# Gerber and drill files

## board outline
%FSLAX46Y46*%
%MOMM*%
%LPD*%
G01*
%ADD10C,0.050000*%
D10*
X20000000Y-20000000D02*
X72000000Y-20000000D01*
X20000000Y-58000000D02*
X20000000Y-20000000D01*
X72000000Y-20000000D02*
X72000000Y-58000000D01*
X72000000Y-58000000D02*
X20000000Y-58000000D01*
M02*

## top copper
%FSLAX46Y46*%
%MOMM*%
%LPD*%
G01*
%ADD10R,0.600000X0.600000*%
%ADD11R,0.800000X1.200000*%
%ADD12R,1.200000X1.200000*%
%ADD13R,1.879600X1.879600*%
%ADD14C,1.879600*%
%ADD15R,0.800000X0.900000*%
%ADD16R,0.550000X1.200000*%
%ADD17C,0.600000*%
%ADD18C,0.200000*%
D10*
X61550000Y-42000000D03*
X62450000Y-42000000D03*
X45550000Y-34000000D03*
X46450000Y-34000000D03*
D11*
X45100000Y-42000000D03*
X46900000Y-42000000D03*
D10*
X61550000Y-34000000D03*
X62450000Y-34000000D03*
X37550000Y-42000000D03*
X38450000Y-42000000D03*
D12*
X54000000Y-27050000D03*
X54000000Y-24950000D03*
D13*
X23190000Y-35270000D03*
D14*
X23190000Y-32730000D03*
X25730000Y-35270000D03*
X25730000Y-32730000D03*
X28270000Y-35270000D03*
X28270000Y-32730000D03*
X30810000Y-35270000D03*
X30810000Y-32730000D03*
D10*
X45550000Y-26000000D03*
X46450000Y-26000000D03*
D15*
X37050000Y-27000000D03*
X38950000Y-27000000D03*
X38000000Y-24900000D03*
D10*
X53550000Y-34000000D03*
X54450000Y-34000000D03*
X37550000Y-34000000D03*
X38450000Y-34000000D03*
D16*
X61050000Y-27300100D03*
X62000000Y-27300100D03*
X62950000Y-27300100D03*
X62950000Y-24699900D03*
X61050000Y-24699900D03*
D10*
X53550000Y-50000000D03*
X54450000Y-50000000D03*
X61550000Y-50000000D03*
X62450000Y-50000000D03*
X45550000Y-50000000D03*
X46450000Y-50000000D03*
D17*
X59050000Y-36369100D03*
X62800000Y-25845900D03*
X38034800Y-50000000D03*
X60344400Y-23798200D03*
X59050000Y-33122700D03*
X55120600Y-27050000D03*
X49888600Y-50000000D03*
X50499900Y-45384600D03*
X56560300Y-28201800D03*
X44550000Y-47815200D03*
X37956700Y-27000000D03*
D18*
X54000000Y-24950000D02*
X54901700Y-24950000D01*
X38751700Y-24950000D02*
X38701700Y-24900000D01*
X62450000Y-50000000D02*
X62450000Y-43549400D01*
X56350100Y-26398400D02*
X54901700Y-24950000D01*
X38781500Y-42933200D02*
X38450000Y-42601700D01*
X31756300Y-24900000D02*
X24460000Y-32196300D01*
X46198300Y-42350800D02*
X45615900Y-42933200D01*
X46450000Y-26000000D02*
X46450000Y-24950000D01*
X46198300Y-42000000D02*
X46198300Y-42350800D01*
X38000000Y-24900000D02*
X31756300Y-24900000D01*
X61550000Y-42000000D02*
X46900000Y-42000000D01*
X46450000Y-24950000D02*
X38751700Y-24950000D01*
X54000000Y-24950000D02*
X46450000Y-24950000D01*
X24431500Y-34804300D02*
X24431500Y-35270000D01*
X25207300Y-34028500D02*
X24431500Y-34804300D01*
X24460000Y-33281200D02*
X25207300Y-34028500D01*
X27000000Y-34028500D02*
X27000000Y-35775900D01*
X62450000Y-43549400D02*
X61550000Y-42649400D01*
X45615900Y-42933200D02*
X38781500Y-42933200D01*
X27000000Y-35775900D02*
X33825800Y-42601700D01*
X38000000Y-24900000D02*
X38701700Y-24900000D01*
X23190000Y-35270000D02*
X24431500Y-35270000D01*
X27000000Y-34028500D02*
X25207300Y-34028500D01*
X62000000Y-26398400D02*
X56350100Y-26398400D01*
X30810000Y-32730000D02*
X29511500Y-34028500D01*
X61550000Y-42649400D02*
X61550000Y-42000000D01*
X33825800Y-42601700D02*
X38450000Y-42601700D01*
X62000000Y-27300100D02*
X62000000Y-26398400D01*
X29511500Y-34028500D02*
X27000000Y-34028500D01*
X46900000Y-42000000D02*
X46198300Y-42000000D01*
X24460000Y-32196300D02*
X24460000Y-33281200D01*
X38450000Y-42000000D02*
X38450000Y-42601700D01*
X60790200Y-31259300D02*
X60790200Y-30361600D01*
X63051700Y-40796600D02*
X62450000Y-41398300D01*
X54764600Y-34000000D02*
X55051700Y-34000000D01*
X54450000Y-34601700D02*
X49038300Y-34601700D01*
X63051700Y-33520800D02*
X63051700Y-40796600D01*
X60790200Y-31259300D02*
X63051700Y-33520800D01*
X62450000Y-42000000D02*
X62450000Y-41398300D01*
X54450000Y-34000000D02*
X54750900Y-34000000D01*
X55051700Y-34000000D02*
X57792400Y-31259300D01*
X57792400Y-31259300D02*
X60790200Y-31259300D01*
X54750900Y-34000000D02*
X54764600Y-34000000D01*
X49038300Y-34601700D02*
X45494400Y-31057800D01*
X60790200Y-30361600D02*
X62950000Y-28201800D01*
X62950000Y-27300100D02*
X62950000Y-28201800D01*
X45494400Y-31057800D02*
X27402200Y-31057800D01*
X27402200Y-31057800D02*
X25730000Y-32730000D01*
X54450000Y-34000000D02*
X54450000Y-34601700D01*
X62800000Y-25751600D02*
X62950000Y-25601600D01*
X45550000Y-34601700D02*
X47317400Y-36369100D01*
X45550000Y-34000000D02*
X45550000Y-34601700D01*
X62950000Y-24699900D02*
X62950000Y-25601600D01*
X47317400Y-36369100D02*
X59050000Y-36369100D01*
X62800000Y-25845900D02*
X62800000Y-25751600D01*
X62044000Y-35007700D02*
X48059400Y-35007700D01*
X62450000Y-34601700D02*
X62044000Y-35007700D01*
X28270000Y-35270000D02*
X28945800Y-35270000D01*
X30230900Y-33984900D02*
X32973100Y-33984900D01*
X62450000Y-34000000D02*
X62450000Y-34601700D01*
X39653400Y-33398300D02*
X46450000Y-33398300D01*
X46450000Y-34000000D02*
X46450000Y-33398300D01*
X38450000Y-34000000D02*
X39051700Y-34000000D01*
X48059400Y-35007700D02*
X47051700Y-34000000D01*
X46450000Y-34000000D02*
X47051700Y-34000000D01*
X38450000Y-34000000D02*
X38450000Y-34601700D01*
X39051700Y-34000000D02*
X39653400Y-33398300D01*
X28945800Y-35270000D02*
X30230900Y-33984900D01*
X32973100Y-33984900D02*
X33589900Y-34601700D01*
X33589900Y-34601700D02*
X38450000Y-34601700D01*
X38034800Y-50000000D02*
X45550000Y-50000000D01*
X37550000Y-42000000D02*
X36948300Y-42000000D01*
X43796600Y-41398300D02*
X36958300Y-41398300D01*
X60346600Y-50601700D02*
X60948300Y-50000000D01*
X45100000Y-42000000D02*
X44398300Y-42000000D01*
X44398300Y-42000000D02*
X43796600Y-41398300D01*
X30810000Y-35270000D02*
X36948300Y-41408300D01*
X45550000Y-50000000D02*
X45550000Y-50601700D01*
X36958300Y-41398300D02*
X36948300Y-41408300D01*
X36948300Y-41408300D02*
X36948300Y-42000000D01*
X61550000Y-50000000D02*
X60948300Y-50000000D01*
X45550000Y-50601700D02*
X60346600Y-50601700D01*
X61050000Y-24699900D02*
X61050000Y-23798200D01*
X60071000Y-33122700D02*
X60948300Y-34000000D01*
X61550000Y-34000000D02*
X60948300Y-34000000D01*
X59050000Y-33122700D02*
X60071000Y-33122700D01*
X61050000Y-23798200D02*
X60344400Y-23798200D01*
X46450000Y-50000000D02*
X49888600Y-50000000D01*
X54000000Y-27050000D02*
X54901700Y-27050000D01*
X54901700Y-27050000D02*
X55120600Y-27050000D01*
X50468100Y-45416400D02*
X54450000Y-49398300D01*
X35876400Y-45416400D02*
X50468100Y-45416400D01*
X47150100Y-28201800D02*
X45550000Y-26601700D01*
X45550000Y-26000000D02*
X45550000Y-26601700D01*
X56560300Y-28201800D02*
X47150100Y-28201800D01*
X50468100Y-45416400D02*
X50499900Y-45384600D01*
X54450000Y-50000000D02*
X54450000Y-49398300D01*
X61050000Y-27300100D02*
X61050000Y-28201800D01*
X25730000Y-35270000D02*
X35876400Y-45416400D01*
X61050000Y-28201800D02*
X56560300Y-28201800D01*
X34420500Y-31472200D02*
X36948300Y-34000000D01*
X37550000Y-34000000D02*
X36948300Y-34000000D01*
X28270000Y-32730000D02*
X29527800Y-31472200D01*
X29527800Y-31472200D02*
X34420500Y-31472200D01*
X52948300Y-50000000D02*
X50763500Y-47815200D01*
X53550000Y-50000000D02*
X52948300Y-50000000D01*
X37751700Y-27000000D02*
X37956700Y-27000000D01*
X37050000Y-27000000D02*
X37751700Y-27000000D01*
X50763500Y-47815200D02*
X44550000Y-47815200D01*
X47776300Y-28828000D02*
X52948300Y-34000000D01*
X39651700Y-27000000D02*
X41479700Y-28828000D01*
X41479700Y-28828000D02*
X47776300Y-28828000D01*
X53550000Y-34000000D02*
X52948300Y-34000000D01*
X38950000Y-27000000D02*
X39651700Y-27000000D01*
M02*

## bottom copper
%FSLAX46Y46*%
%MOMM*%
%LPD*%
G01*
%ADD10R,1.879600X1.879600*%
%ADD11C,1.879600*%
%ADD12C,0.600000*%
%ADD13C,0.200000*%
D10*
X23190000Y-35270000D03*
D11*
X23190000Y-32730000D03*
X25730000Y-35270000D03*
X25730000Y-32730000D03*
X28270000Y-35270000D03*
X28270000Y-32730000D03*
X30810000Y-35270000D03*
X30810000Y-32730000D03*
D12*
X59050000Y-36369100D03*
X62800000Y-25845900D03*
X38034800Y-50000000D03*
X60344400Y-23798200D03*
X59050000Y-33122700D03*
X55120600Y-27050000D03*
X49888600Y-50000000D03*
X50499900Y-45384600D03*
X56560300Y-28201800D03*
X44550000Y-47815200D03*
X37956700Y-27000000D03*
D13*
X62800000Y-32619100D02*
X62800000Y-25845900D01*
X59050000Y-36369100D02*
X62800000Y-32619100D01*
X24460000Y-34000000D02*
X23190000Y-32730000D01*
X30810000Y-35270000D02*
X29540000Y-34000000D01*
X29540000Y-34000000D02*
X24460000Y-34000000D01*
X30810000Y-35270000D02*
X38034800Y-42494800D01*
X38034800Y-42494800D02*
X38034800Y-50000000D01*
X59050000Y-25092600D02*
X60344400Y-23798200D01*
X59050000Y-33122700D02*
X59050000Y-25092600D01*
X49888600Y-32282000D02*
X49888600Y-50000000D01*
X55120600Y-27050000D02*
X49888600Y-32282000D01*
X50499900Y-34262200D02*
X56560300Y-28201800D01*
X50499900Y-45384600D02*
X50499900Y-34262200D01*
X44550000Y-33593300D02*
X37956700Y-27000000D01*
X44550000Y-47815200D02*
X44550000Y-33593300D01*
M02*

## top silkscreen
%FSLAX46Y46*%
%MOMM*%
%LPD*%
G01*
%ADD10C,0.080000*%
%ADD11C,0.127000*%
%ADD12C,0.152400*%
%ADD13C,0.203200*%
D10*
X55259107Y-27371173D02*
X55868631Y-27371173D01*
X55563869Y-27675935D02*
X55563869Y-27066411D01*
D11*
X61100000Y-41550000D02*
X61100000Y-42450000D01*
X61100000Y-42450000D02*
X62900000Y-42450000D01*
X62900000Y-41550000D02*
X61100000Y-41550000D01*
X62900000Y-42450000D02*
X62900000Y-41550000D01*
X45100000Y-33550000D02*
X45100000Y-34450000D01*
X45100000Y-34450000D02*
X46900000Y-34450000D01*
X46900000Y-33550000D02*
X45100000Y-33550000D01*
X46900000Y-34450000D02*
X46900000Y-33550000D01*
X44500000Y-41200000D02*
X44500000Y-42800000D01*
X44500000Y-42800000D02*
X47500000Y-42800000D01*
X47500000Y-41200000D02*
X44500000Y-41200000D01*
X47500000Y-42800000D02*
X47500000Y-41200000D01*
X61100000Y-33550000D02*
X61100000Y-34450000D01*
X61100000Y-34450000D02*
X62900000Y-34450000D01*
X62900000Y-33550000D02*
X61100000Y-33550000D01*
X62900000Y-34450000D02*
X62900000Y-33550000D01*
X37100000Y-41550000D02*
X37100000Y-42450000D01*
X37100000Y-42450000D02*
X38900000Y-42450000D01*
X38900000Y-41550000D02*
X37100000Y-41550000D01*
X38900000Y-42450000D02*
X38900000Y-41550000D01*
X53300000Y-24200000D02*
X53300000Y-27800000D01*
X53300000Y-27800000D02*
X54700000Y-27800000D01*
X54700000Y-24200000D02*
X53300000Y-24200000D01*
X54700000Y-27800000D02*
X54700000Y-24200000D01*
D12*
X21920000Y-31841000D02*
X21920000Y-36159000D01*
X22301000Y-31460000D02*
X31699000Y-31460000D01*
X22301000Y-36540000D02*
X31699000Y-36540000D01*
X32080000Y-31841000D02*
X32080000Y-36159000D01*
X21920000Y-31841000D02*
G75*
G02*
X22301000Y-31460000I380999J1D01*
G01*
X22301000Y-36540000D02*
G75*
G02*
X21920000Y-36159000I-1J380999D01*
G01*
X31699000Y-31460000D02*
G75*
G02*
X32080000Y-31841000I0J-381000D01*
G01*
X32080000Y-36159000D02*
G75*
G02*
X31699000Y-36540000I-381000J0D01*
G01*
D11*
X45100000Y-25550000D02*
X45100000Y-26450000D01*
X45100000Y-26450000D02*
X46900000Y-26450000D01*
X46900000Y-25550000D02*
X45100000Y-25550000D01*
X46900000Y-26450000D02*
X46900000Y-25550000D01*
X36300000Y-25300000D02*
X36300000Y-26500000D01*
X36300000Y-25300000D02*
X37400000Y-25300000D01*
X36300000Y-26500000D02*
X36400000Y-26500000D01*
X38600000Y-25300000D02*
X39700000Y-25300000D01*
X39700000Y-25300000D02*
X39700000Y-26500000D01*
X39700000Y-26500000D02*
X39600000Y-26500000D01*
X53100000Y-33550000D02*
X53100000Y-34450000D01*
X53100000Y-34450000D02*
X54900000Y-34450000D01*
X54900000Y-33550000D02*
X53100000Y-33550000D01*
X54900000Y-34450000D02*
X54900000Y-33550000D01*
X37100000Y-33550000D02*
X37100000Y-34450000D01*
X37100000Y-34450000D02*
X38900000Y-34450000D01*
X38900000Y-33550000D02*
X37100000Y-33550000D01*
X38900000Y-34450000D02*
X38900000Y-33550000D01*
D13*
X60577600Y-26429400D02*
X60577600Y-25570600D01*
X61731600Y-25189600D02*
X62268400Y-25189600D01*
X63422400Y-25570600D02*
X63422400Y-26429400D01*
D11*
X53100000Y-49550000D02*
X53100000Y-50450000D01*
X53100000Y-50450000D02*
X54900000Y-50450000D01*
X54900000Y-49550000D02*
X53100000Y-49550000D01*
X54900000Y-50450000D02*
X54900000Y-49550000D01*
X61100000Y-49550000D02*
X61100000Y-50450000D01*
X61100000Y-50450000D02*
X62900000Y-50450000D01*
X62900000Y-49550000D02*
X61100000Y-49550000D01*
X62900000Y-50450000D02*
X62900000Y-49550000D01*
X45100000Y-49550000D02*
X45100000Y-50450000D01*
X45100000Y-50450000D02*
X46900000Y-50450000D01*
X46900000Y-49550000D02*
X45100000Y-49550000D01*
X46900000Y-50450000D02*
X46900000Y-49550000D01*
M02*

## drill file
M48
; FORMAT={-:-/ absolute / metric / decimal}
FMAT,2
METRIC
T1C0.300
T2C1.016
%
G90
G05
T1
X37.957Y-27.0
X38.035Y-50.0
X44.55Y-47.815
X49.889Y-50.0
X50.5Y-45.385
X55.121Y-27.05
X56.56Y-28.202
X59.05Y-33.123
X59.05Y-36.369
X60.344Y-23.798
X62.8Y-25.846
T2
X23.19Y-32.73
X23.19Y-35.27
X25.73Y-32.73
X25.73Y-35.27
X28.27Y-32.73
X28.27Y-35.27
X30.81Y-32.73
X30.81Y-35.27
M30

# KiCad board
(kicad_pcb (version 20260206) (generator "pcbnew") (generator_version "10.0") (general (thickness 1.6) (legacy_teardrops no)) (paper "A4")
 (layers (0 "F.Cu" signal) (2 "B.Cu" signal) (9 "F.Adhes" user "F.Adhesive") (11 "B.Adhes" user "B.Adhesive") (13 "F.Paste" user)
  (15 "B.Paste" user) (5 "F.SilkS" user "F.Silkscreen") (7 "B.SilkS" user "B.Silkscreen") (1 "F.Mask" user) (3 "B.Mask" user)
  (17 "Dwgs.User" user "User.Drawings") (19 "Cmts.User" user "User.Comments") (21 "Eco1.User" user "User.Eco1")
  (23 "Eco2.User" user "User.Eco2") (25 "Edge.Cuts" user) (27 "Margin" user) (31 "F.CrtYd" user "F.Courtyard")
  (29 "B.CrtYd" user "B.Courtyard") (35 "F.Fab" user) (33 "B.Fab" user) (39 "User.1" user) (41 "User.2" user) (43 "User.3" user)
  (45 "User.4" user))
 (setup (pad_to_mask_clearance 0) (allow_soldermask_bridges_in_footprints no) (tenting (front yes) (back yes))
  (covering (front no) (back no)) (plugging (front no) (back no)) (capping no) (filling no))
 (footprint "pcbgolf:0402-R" (layer "F.Cu") (at 62 42)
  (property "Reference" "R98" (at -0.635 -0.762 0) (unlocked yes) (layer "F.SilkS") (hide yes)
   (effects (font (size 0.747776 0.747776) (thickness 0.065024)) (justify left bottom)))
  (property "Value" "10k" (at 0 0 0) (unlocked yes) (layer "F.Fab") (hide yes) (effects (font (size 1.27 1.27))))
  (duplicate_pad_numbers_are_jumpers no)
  (fp_line (start -0.9 -0.45) (end -0.9 0.45) (stroke (width 0.127) (type solid)) (layer "F.SilkS"))
  (fp_line (start -0.9 0.45) (end 0.9 0.45) (stroke (width 0.127) (type solid)) (layer "F.SilkS"))
  (fp_line (start 0.9 -0.45) (end -0.9 -0.45) (stroke (width 0.127) (type solid)) (layer "F.SilkS"))
  (fp_line (start 0.9 0.45) (end 0.9 -0.45) (stroke (width 0.127) (type solid)) (layer "F.SilkS"))
  (pad "1" smd rect (at -0.45 0) (size 0.6 0.6) (layers "F.Cu" "F.Mask" "F.Paste") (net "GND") (solder_mask_margin 0.0508)
   (solder_paste_margin 0) (thermal_bridge_angle 0))
  (pad "2" smd rect (at 0.45 0) (size 0.6 0.6) (layers "F.Cu" "F.Mask" "F.Paste") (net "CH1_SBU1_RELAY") (solder_mask_margin 0.0508)
   (solder_paste_margin 0) (thermal_bridge_angle 0)))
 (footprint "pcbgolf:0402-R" (layer "F.Cu") (at 46 34)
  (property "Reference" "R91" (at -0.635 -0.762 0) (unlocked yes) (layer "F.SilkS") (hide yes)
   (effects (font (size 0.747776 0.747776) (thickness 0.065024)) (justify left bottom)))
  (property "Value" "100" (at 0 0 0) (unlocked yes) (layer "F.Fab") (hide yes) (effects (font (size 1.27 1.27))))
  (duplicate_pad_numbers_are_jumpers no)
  (fp_line (start -0.9 -0.45) (end -0.9 0.45) (stroke (width 0.127) (type solid)) (layer "F.SilkS"))
  (fp_line (start -0.9 0.45) (end 0.9 0.45) (stroke (width 0.127) (type solid)) (layer "F.SilkS"))
  (fp_line (start 0.9 -0.45) (end -0.9 -0.45) (stroke (width 0.127) (type solid)) (layer "F.SilkS"))
  (fp_line (start 0.9 0.45) (end 0.9 -0.45) (stroke (width 0.127) (type solid)) (layer "F.SilkS"))
  (pad "1" smd rect (at -0.45 0) (size 0.6 0.6) (layers "F.Cu" "F.Mask" "F.Paste") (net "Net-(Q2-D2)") (solder_mask_margin 0.0508)
   (solder_paste_margin 0) (thermal_bridge_angle 0))
  (pad "2" smd rect (at 0.45 0) (size 0.6 0.6) (layers "F.Cu" "F.Mask" "F.Paste") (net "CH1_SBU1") (solder_mask_margin 0.0508)
   (solder_paste_margin 0) (thermal_bridge_angle 0)))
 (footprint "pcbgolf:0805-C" (layer "F.Cu") (at 46 42)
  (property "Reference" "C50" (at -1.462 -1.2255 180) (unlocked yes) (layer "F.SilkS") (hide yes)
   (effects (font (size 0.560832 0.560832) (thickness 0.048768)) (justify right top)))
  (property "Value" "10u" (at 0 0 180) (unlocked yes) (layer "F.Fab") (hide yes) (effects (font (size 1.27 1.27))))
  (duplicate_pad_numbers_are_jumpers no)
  (fp_line (start -1.5 -0.8) (end -1.5 0.8) (stroke (width 0.127) (type solid)) (layer "F.SilkS"))
  (fp_line (start -1.5 0.8) (end 1.5 0.8) (stroke (width 0.127) (type solid)) (layer "F.SilkS"))
  (fp_line (start 1.5 -0.8) (end -1.5 -0.8) (stroke (width 0.127) (type solid)) (layer "F.SilkS"))
  (fp_line (start 1.5 0.8) (end 1.5 -0.8) (stroke (width 0.127) (type solid)) (layer "F.SilkS"))
  (pad "1" smd rect (at -0.9 0) (size 0.8 1.2) (layers "F.Cu" "F.Mask" "F.Paste") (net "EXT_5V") (solder_mask_margin 0.0508)
   (solder_paste_margin 0) (thermal_bridge_angle 0))
  (pad "2" smd rect (at 0.9 0) (size 0.8 1.2) (layers "F.Cu" "F.Mask" "F.Paste") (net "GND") (solder_mask_margin 0.0508)
   (solder_paste_margin 0) (thermal_bridge_angle 0)))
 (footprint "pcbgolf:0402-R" (layer "F.Cu") (at 62 34)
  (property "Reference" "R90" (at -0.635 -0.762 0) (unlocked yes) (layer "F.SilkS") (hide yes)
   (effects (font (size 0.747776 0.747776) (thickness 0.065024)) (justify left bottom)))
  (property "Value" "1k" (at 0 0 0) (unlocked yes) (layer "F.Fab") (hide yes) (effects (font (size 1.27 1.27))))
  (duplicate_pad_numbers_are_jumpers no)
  (fp_line (start -0.9 -0.45) (end -0.9 0.45) (stroke (width 0.127) (type solid)) (layer "F.SilkS"))
  (fp_line (start -0.9 0.45) (end 0.9 0.45) (stroke (width 0.127) (type solid)) (layer "F.SilkS"))
  (fp_line (start 0.9 -0.45) (end -0.9 -0.45) (stroke (width 0.127) (type solid)) (layer "F.SilkS"))
  (fp_line (start 0.9 0.45) (end 0.9 -0.45) (stroke (width 0.127) (type solid)) (layer "F.SilkS"))
  (pad "1" smd rect (at -0.45 0) (size 0.6 0.6) (layers "F.Cu" "F.Mask" "F.Paste") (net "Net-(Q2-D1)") (solder_mask_margin 0.0508)
   (solder_paste_margin 0) (thermal_bridge_angle 0))
  (pad "2" smd rect (at 0.45 0) (size 0.6 0.6) (layers "F.Cu" "F.Mask" "F.Paste") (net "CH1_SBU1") (solder_mask_margin 0.0508)
   (solder_paste_margin 0) (thermal_bridge_angle 0)))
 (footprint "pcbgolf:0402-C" (layer "F.Cu") (at 38 42)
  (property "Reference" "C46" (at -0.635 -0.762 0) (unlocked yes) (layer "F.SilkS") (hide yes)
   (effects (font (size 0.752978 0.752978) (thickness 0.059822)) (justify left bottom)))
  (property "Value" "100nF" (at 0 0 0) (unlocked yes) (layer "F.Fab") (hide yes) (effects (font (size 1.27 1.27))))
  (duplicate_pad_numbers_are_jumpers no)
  (fp_line (start -0.9 -0.45) (end -0.9 0.45) (stroke (width 0.127) (type solid)) (layer "F.SilkS"))
  (fp_line (start -0.9 0.45) (end 0.9 0.45) (stroke (width 0.127) (type solid)) (layer "F.SilkS"))
  (fp_line (start 0.9 -0.45) (end -0.9 -0.45) (stroke (width 0.127) (type solid)) (layer "F.SilkS"))
  (fp_line (start 0.9 0.45) (end 0.9 -0.45) (stroke (width 0.127) (type solid)) (layer "F.SilkS"))
  (pad "1" smd rect (at -0.45 0) (size 0.6 0.6) (layers "F.Cu" "F.Mask" "F.Paste") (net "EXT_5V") (solder_mask_margin 0.0508)
   (solder_paste_margin 0) (thermal_bridge_angle 0))
  (pad "2" smd rect (at 0.45 0) (size 0.6 0.6) (layers "F.Cu" "F.Mask" "F.Paste") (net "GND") (solder_mask_margin 0.0508)
   (solder_paste_margin 0) (thermal_bridge_angle 0)))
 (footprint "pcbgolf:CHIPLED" (layer "F.Cu") (at 54 26)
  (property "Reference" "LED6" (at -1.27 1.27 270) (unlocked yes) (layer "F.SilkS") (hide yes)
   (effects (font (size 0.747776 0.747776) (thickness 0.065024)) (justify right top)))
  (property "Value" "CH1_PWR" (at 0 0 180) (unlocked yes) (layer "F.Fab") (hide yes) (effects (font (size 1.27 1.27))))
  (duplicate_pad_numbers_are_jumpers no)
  (fp_line (start -0.7 -1.8) (end -0.7 1.8) (stroke (width 0.127) (type solid)) (layer "F.SilkS"))
  (fp_line (start -0.7 1.8) (end 0.7 1.8) (stroke (width 0.127) (type solid)) (layer "F.SilkS"))
  (fp_line (start 0.7 -1.8) (end -0.7 -1.8) (stroke (width 0.127) (type solid)) (layer "F.SilkS"))
  (fp_line (start 0.7 1.8) (end 0.7 -1.8) (stroke (width 0.127) (type solid)) (layer "F.SilkS"))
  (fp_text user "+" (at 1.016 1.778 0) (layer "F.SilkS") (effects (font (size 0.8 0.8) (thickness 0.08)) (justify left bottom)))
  (pad "A" smd rect (at 0 1.05) (size 1.2 1.2) (layers "F.Cu" "F.Mask" "F.Paste") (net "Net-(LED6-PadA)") (solder_mask_margin 0.0508)
   (solder_paste_margin 0) (thermal_bridge_angle 0))
  (pad "C" smd rect (at 0 -1.05) (size 1.2 1.2) (layers "F.Cu" "F.Mask" "F.Paste") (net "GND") (solder_mask_margin 0.0508)
   (solder_paste_margin 0) (thermal_bridge_angle 0)))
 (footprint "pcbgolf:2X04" (layer "F.Cu") (at 27 34)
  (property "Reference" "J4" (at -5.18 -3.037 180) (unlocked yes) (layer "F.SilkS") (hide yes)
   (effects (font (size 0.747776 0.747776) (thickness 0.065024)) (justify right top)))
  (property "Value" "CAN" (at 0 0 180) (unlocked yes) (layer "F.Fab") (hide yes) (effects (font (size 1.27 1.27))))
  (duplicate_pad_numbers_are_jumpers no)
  (fp_line (start -5.08 -2.159) (end -5.08 2.159) (stroke (width 0.1524) (type solid)) (layer "F.SilkS"))
  (fp_line (start -4.699 -2.54) (end 4.699 -2.54) (stroke (width 0.1524) (type solid)) (layer "F.SilkS"))
  (fp_line (start -4.699 2.54) (end 4.699 2.54) (stroke (width 0.1524) (type solid)) (layer "F.SilkS"))
  (fp_line (start 5.08 -2.159) (end 5.08 2.159) (stroke (width 0.1524) (type solid)) (layer "F.SilkS"))
  (fp_arc (start -5.08 -2.159) (mid -4.968408 -2.428408) (end -4.699 -2.54) (stroke (width 0.1524) (type solid)) (layer "F.SilkS"))
  (fp_arc (start -4.699 2.54) (mid -4.968408 2.428408) (end -5.08 2.159) (stroke (width 0.1524) (type solid)) (layer "F.SilkS"))
  (fp_arc (start 4.699 -2.54) (mid 4.968408 -2.428408) (end 5.08 -2.159) (stroke (width 0.1524) (type solid)) (layer "F.SilkS"))
  (fp_arc (start 5.08 2.159) (mid 4.968408 2.428408) (end 4.699 2.54) (stroke (width 0.1524) (type solid)) (layer "F.SilkS"))
  (pad "1" thru_hole rect (at -3.81 1.27 90) (size 1.8796 1.8796) (drill 1.016) (layers "*.Cu" "*.Mask") (remove_unused_layers no)
   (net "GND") (solder_mask_margin 0.0508) (thermal_bridge_angle 0))
  (pad "2" thru_hole circle (at -3.81 -1.27 90) (size 1.8796 1.8796) (drill 1.016) (layers "*.Cu" "*.Mask") (remove_unused_layers no)
   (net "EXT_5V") (solder_mask_margin 0.0508) (thermal_bridge_angle 0))
  (pad "3" thru_hole circle (at -1.27 1.27 90) (size 1.8796 1.8796) (drill 1.016) (layers "*.Cu" "*.Mask") (remove_unused_layers no)
   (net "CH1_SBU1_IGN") (solder_mask_margin 0.0508) (thermal_bridge_angle 0))
  (pad "4" thru_hole circle (at -1.27 -1.27 90) (size 1.8796 1.8796) (drill 1.016) (layers "*.Cu" "*.Mask") (remove_unused_layers no)
   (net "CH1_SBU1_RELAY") (solder_mask_margin 0.0508) (thermal_bridge_angle 0))
  (pad "5" thru_hole circle (at 1.27 1.27 90) (size 1.8796 1.8796) (drill 1.016) (layers "*.Cu" "*.Mask") (remove_unused_layers no)
   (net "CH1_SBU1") (solder_mask_margin 0.0508) (thermal_bridge_angle 0))
  (pad "6" thru_hole circle (at 1.27 -1.27 90) (size 1.8796 1.8796) (drill 1.016) (layers "*.Cu" "*.Mask") (remove_unused_layers no)
   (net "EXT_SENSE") (solder_mask_margin 0.0508) (thermal_bridge_angle 0))
  (pad "7" thru_hole circle (at 3.81 1.27 90) (size 1.8796 1.8796) (drill 1.016) (layers "*.Cu" "*.Mask") (remove_unused_layers no)
   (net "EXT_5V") (solder_mask_margin 0.0508) (thermal_bridge_angle 0))
  (pad "8" thru_hole circle (at 3.81 -1.27 90) (size 1.8796 1.8796) (drill 1.016) (layers "*.Cu" "*.Mask") (remove_unused_layers no)
   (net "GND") (solder_mask_margin 0.0508) (thermal_bridge_angle 0)))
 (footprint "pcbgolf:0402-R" (layer "F.Cu") (at 46 26)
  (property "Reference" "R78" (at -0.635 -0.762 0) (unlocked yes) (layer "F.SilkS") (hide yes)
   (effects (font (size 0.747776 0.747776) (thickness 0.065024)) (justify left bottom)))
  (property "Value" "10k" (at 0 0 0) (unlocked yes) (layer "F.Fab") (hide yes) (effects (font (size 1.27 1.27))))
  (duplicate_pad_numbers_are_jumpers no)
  (fp_line (start -0.9 -0.45) (end -0.9 0.45) (stroke (width 0.127) (type solid)) (layer "F.SilkS"))
  (fp_line (start -0.9 0.45) (end 0.9 0.45) (stroke (width 0.127) (type solid)) (layer "F.SilkS"))
  (fp_line (start 0.9 -0.45) (end -0.9 -0.45) (stroke (width 0.127) (type solid)) (layer "F.SilkS"))
  (fp_line (start 0.9 0.45) (end 0.9 -0.45) (stroke (width 0.127) (type solid)) (layer "F.SilkS"))
  (pad "1" smd rect (at -0.45 0) (size 0.6 0.6) (layers "F.Cu" "F.Mask" "F.Paste") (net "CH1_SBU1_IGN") (solder_mask_margin 0.0508)
   (solder_paste_margin 0) (thermal_bridge_angle 0))
  (pad "2" smd rect (at 0.45 0) (size 0.6 0.6) (layers "F.Cu" "F.Mask" "F.Paste") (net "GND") (solder_mask_margin 0.0508)
   (solder_paste_margin 0) (thermal_bridge_angle 0)))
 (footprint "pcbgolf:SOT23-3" (layer "F.Cu") (at 38 26)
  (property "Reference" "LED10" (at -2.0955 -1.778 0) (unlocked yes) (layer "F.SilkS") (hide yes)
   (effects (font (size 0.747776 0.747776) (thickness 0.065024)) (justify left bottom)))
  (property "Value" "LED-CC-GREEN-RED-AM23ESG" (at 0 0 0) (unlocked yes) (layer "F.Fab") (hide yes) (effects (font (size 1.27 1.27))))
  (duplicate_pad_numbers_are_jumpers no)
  (fp_line (start -1.7 -0.7) (end -1.7 0.5) (stroke (width 0.127) (type solid)) (layer "F.SilkS"))
  (fp_line (start -1.7 -0.7) (end -0.6 -0.7) (stroke (width 0.127) (type solid)) (layer "F.SilkS"))
  (fp_line (start -1.7 0.5) (end -1.6 0.5) (stroke (width 0.127) (type solid)) (layer "F.SilkS"))
  (fp_line (start 0.6 -0.7) (end 1.7 -0.7) (stroke (width 0.127) (type solid)) (layer "F.SilkS"))
  (fp_line (start 1.7 -0.7) (end 1.7 0.5) (stroke (width 0.127) (type solid)) (layer "F.SilkS"))
  (fp_line (start 1.7 0.5) (end 1.6 0.5) (stroke (width 0.127) (type solid)) (layer "F.SilkS"))
  (pad "1" smd rect (at -0.95 1) (size 0.8 0.9) (layers "F.Cu" "F.Mask" "F.Paste") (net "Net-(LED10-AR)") (solder_mask_margin 0.0508)
   (solder_paste_margin 0) (thermal_bridge_angle 0))
  (pad "2" smd rect (at 0.95 1) (size 0.8 0.9) (layers "F.Cu" "F.Mask" "F.Paste") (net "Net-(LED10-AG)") (solder_mask_margin 0.0508)
   (solder_paste_margin 0) (thermal_bridge_angle 0))
  (pad "3" smd rect (at 0 -1.1) (size 0.8 0.9) (layers "F.Cu" "F.Mask" "F.Paste") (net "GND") (solder_mask_margin 0.0508)
   (solder_paste_margin 0) (thermal_bridge_angle 0)))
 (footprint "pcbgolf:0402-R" (layer "F.Cu") (at 54 34)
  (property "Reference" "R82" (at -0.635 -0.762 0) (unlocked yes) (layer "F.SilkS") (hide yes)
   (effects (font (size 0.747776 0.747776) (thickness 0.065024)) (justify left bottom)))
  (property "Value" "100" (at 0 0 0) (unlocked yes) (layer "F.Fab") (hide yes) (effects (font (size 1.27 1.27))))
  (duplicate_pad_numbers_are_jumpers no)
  (fp_line (start -0.9 -0.45) (end -0.9 0.45) (stroke (width 0.127) (type solid)) (layer "F.SilkS"))
  (fp_line (start -0.9 0.45) (end 0.9 0.45) (stroke (width 0.127) (type solid)) (layer "F.SilkS"))
  (fp_line (start 0.9 -0.45) (end -0.9 -0.45) (stroke (width 0.127) (type solid)) (layer "F.SilkS"))
  (fp_line (start 0.9 0.45) (end 0.9 -0.45) (stroke (width 0.127) (type solid)) (layer "F.SilkS"))
  (pad "1" smd rect (at -0.45 0) (size 0.6 0.6) (layers "F.Cu" "F.Mask" "F.Paste") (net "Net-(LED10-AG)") (solder_mask_margin 0.0508)
   (solder_paste_margin 0) (thermal_bridge_angle 0))
  (pad "2" smd rect (at 0.45 0) (size 0.6 0.6) (layers "F.Cu" "F.Mask" "F.Paste") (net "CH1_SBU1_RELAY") (solder_mask_margin 0.0508)
   (solder_paste_margin 0) (thermal_bridge_angle 0)))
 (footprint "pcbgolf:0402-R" (layer "F.Cu") (at 38 34)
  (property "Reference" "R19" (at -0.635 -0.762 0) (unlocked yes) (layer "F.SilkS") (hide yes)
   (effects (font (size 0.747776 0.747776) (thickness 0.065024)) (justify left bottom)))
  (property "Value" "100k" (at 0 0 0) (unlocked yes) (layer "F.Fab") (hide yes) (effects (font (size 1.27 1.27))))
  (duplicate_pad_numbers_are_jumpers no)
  (fp_line (start -0.9 -0.45) (end -0.9 0.45) (stroke (width 0.127) (type solid)) (layer "F.SilkS"))
  (fp_line (start -0.9 0.45) (end 0.9 0.45) (stroke (width 0.127) (type solid)) (layer "F.SilkS"))
  (fp_line (start 0.9 -0.45) (end -0.9 -0.45) (stroke (width 0.127) (type solid)) (layer "F.SilkS"))
  (fp_line (start 0.9 0.45) (end 0.9 -0.45) (stroke (width 0.127) (type solid)) (layer "F.SilkS"))
  (pad "1" smd rect (at -0.45 0) (size 0.6 0.6) (layers "F.Cu" "F.Mask" "F.Paste") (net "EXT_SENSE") (solder_mask_margin 0.0508)
   (solder_paste_margin 0) (thermal_bridge_angle 0))
  (pad "2" smd rect (at 0.45 0) (size 0.6 0.6) (layers "F.Cu" "F.Mask" "F.Paste") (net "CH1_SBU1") (solder_mask_margin 0.0508)
   (solder_paste_margin 0) (thermal_bridge_angle 0)))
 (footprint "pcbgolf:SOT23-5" (layer "F.Cu") (at 62 26)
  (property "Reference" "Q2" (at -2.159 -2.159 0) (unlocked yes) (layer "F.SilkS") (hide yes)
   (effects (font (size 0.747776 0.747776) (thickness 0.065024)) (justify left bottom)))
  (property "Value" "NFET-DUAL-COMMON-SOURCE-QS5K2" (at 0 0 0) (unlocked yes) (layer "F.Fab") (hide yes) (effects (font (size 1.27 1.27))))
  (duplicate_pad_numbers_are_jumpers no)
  (fp_line (start -1.4224 0.4294) (end -1.4224 -0.4294) (stroke (width 0.2032) (type solid)) (layer "F.SilkS"))
  (fp_line (start -0.2684 -0.8104) (end 0.2684 -0.8104) (stroke (width 0.2032) (type solid)) (layer "F.SilkS"))
  (fp_line (start 1.4224 -0.4294) (end 1.4224 0.4294) (stroke (width 0.2032) (type solid)) (layer "F.SilkS"))
  (pad "1" smd rect (at -0.95 1.3001) (size 0.55 1.2) (layers "F.Cu" "F.Mask" "F.Paste") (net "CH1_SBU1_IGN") (solder_mask_margin 0.0508)
   (solder_paste_margin 0) (thermal_bridge_angle 0))
  (pad "2" smd rect (at 0 1.3001) (size 0.55 1.2) (layers "F.Cu" "F.Mask" "F.Paste") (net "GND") (solder_mask_margin 0.0508)
   (solder_paste_margin 0) (thermal_bridge_angle 0))
  (pad "3" smd rect (at 0.95 1.3001) (size 0.55 1.2) (layers "F.Cu" "F.Mask" "F.Paste") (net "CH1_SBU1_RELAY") (solder_mask_margin 0.0508)
   (solder_paste_margin 0) (thermal_bridge_angle 0))
  (pad "4" smd rect (at 0.95 -1.3001) (size 0.55 1.2) (layers "F.Cu" "F.Mask" "F.Paste") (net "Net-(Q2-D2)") (solder_mask_margin 0.0508)
   (solder_paste_margin 0) (thermal_bridge_angle 0))
  (pad "5" smd rect (at -0.95 -1.3001) (size 0.55 1.2) (layers "F.Cu" "F.Mask" "F.Paste") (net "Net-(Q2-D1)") (solder_mask_margin 0.0508)
   (solder_paste_margin 0) (thermal_bridge_angle 0)))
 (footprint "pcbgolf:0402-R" (layer "F.Cu") (at 54 50)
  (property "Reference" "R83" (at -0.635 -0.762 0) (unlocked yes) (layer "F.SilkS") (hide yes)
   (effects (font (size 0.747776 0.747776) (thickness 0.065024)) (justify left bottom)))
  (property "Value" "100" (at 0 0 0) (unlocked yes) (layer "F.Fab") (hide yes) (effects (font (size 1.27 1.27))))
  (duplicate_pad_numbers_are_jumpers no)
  (fp_line (start -0.9 -0.45) (end -0.9 0.45) (stroke (width 0.127) (type solid)) (layer "F.SilkS"))
  (fp_line (start -0.9 0.45) (end 0.9 0.45) (stroke (width 0.127) (type solid)) (layer "F.SilkS"))
  (fp_line (start 0.9 -0.45) (end -0.9 -0.45) (stroke (width 0.127) (type solid)) (layer "F.SilkS"))
  (fp_line (start 0.9 0.45) (end 0.9 -0.45) (stroke (width 0.127) (type solid)) (layer "F.SilkS"))
  (pad "1" smd rect (at -0.45 0) (size 0.6 0.6) (layers "F.Cu" "F.Mask" "F.Paste") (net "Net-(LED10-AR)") (solder_mask_margin 0.0508)
   (solder_paste_margin 0) (thermal_bridge_angle 0))
  (pad "2" smd rect (at 0.45 0) (size 0.6 0.6) (layers "F.Cu" "F.Mask" "F.Paste") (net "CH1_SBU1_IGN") (solder_mask_margin 0.0508)
   (solder_paste_margin 0) (thermal_bridge_angle 0)))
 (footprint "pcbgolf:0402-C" (layer "F.Cu") (at 62 50)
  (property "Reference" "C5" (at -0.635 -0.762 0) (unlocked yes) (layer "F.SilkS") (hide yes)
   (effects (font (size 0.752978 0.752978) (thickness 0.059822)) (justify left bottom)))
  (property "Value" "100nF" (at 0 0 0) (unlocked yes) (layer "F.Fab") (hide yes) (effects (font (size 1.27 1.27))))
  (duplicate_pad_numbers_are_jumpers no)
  (fp_line (start -0.9 -0.45) (end -0.9 0.45) (stroke (width 0.127) (type solid)) (layer "F.SilkS"))
  (fp_line (start -0.9 0.45) (end 0.9 0.45) (stroke (width 0.127) (type solid)) (layer "F.SilkS"))
  (fp_line (start 0.9 -0.45) (end -0.9 -0.45) (stroke (width 0.127) (type solid)) (layer "F.SilkS"))
  (fp_line (start 0.9 0.45) (end 0.9 -0.45) (stroke (width 0.127) (type solid)) (layer "F.SilkS"))
  (pad "1" smd rect (at -0.45 0) (size 0.6 0.6) (layers "F.Cu" "F.Mask" "F.Paste") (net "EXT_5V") (solder_mask_margin 0.0508)
   (solder_paste_margin 0) (thermal_bridge_angle 0))
  (pad "2" smd rect (at 0.45 0) (size 0.6 0.6) (layers "F.Cu" "F.Mask" "F.Paste") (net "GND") (solder_mask_margin 0.0508)
   (solder_paste_margin 0) (thermal_bridge_angle 0)))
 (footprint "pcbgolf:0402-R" (layer "F.Cu") (at 46 50)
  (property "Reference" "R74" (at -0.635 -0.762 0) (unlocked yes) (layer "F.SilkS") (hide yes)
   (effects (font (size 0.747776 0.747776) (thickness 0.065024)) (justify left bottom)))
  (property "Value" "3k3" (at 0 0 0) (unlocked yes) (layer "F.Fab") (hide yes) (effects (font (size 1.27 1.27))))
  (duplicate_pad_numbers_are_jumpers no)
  (fp_line (start -0.9 -0.45) (end -0.9 0.45) (stroke (width 0.127) (type solid)) (layer "F.SilkS"))
  (fp_line (start -0.9 0.45) (end 0.9 0.45) (stroke (width 0.127) (type solid)) (layer "F.SilkS"))
  (fp_line (start 0.9 -0.45) (end -0.9 -0.45) (stroke (width 0.127) (type solid)) (layer "F.SilkS"))
  (fp_line (start 0.9 0.45) (end 0.9 -0.45) (stroke (width 0.127) (type solid)) (layer "F.SilkS"))
  (pad "1" smd rect (at -0.45 0) (size 0.6 0.6) (layers "F.Cu" "F.Mask" "F.Paste") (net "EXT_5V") (solder_mask_margin 0.0508)
   (solder_paste_margin 0) (thermal_bridge_angle 0))
  (pad "2" smd rect (at 0.45 0) (size 0.6 0.6) (layers "F.Cu" "F.Mask" "F.Paste") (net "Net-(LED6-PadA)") (solder_mask_margin 0.0508)
   (solder_paste_margin 0) (thermal_bridge_angle 0)))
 (gr_line (start 20 20) (end 72 20) (stroke (width 0.05) (type default)) (layer "Edge.Cuts"))
 (gr_line (start 20 58) (end 20 20) (stroke (width 0.05) (type default)) (layer "Edge.Cuts"))
 (gr_line (start 72 20) (end 72 58) (stroke (width 0.05) (type default)) (layer "Edge.Cuts"))
 (gr_line (start 72 58) (end 20 58) (stroke (width 0.05) (type default)) (layer "Edge.Cuts"))
 (segment (start 54 24.95) (end 54.9017 24.95) (width 0.2) (layer "F.Cu") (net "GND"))
 (segment (start 38.7517 24.95) (end 38.7017 24.9) (width 0.2) (layer "F.Cu") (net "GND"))
 (segment (start 62.45 50) (end 62.45 43.5494) (width 0.2) (layer "F.Cu") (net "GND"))
 (segment (start 56.3501 26.3984) (end 54.9017 24.95) (width 0.2) (layer "F.Cu") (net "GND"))
 (segment (start 38.7815 42.9332) (end 38.45 42.6017) (width 0.2) (layer "F.Cu") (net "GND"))
 (segment (start 31.7563 24.9) (end 24.46 32.1963) (width 0.2) (layer "F.Cu") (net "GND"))
 (segment (start 46.1983 42.3508) (end 45.6159 42.9332) (width 0.2) (layer "F.Cu") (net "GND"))
 (segment (start 46.45 26) (end 46.45 24.95) (width 0.2) (layer "F.Cu") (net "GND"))
 (segment (start 46.1983 42) (end 46.1983 42.3508) (width 0.2) (layer "F.Cu") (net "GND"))
 (segment (start 38 24.9) (end 31.7563 24.9) (width 0.2) (layer "F.Cu") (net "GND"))
 (segment (start 61.55 42) (end 46.9 42) (width 0.2) (layer "F.Cu") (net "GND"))
 (segment (start 46.45 24.95) (end 38.7517 24.95) (width 0.2) (layer "F.Cu") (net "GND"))
 (segment (start 54 24.95) (end 46.45 24.95) (width 0.2) (layer "F.Cu") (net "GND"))
 (segment (start 24.4315 34.8043) (end 24.4315 35.27) (width 0.2) (layer "F.Cu") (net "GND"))
 (segment (start 25.2073 34.0285) (end 24.4315 34.8043) (width 0.2) (layer "F.Cu") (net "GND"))
 (segment (start 24.46 33.2812) (end 25.2073 34.0285) (width 0.2) (layer "F.Cu") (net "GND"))
 (segment (start 27 34.0285) (end 27 35.7759) (width 0.2) (layer "F.Cu") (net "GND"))
 (segment (start 62.45 43.5494) (end 61.55 42.6494) (width 0.2) (layer "F.Cu") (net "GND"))
 (segment (start 45.6159 42.9332) (end 38.7815 42.9332) (width 0.2) (layer "F.Cu") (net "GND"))
 (segment (start 27 35.7759) (end 33.8258 42.6017) (width 0.2) (layer "F.Cu") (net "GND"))
 (segment (start 38 24.9) (end 38.7017 24.9) (width 0.2) (layer "F.Cu") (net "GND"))
 (segment (start 23.19 35.27) (end 24.4315 35.27) (width 0.2) (layer "F.Cu") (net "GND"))
 (segment (start 27 34.0285) (end 25.2073 34.0285) (width 0.2) (layer "F.Cu") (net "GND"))
 (segment (start 62 26.3984) (end 56.3501 26.3984) (width 0.2) (layer "F.Cu") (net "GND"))
 (segment (start 30.81 32.73) (end 29.5115 34.0285) (width 0.2) (layer "F.Cu") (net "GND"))
 (segment (start 61.55 42.6494) (end 61.55 42) (width 0.2) (layer "F.Cu") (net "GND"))
 (segment (start 33.8258 42.6017) (end 38.45 42.6017) (width 0.2) (layer "F.Cu") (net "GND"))
 (segment (start 62 27.3001) (end 62 26.3984) (width 0.2) (layer "F.Cu") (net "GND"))
 (segment (start 29.5115 34.0285) (end 27 34.0285) (width 0.2) (layer "F.Cu") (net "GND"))
 (segment (start 46.9 42) (end 46.1983 42) (width 0.2) (layer "F.Cu") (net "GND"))
 (segment (start 24.46 32.1963) (end 24.46 33.2812) (width 0.2) (layer "F.Cu") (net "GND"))
 (segment (start 38.45 42) (end 38.45 42.6017) (width 0.2) (layer "F.Cu") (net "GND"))
 (segment (start 60.7902 31.2593) (end 60.7902 30.3616) (width 0.2) (layer "F.Cu") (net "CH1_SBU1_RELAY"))
 (segment (start 63.0517 40.7966) (end 62.45 41.3983) (width 0.2) (layer "F.Cu") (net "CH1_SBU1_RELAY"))
 (segment (start 54.7646 34) (end 55.0517 34) (width 0.2) (layer "F.Cu") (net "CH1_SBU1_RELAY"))
 (segment (start 54.45 34.6017) (end 49.0383 34.6017) (width 0.2) (layer "F.Cu") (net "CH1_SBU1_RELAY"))
 (segment (start 63.0517 33.5208) (end 63.0517 40.7966) (width 0.2) (layer "F.Cu") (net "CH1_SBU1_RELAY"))
 (segment (start 60.7902 31.2593) (end 63.0517 33.5208) (width 0.2) (layer "F.Cu") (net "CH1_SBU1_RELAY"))
 (segment (start 62.45 42) (end 62.45 41.3983) (width 0.2) (layer "F.Cu") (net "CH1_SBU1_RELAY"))
 (segment (start 54.45 34) (end 54.7509 34) (width 0.2) (layer "F.Cu") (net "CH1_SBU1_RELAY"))
 (segment (start 55.0517 34) (end 57.7924 31.2593) (width 0.2) (layer "F.Cu") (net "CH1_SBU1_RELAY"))
 (segment (start 57.7924 31.2593) (end 60.7902 31.2593) (width 0.2) (layer "F.Cu") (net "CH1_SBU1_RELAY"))
 (segment (start 54.7509 34) (end 54.7646 34) (width 0.2) (layer "F.Cu") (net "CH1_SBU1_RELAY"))
 (segment (start 49.0383 34.6017) (end 45.4944 31.0578) (width 0.2) (layer "F.Cu") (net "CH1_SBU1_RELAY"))
 (segment (start 60.7902 30.3616) (end 62.95 28.2018) (width 0.2) (layer "F.Cu") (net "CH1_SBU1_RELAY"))
 (segment (start 62.95 27.3001) (end 62.95 28.2018) (width 0.2) (layer "F.Cu") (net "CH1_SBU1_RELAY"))
 (segment (start 45.4944 31.0578) (end 27.4022 31.0578) (width 0.2) (layer "F.Cu") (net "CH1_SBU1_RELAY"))
 (segment (start 27.4022 31.0578) (end 25.73 32.73) (width 0.2) (layer "F.Cu") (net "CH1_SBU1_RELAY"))
 (segment (start 54.45 34) (end 54.45 34.6017) (width 0.2) (layer "F.Cu") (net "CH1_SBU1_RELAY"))
 (segment (start 62.8 25.7516) (end 62.95 25.6016) (width 0.2) (layer "F.Cu") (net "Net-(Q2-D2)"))
 (segment (start 45.55 34.6017) (end 47.3174 36.3691) (width 0.2) (layer "F.Cu") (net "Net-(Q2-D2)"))
 (segment (start 45.55 34) (end 45.55 34.6017) (width 0.2) (layer "F.Cu") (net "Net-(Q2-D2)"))
 (segment (start 62.95 24.6999) (end 62.95 25.6016) (width 0.2) (layer "F.Cu") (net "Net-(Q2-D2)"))
 (segment (start 47.3174 36.3691) (end 59.05 36.3691) (width 0.2) (layer "F.Cu") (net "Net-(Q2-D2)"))
 (segment (start 62.8 25.8459) (end 62.8 25.7516) (width 0.2) (layer "F.Cu") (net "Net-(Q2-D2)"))
 (via (at 59.05 36.3691) (size 0.6) (drill 0.3) (layers "F.Cu" "B.Cu") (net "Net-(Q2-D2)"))
 (via (at 62.8 25.8459) (size 0.6) (drill 0.3) (layers "F.Cu" "B.Cu") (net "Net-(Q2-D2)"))
 (segment (start 62.8 32.6191) (end 62.8 25.8459) (width 0.2) (layer "B.Cu") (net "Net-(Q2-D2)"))
 (segment (start 59.05 36.3691) (end 62.8 32.6191) (width 0.2) (layer "B.Cu") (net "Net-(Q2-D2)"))
 (segment (start 62.044 35.0077) (end 48.0594 35.0077) (width 0.2) (layer "F.Cu") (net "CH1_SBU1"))
 (segment (start 62.45 34.6017) (end 62.044 35.0077) (width 0.2) (layer "F.Cu") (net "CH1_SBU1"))
 (segment (start 28.27 35.27) (end 28.9458 35.27) (width 0.2) (layer "F.Cu") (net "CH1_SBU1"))
 (segment (start 30.2309 33.9849) (end 32.9731 33.9849) (width 0.2) (layer "F.Cu") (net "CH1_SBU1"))
 (segment (start 62.45 34) (end 62.45 34.6017) (width 0.2) (layer "F.Cu") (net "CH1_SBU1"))
 (segment (start 39.6534 33.3983) (end 46.45 33.3983) (width 0.2) (layer "F.Cu") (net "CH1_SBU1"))
 (segment (start 46.45 34) (end 46.45 33.3983) (width 0.2) (layer "F.Cu") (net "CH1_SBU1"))
 (segment (start 38.45 34) (end 39.0517 34) (width 0.2) (layer "F.Cu") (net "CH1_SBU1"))
 (segment (start 48.0594 35.0077) (end 47.0517 34) (width 0.2) (layer "F.Cu") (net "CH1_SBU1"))
 (segment (start 46.45 34) (end 47.0517 34) (width 0.2) (layer "F.Cu") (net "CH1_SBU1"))
 (segment (start 38.45 34) (end 38.45 34.6017) (width 0.2) (layer "F.Cu") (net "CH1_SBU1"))
 (segment (start 39.0517 34) (end 39.6534 33.3983) (width 0.2) (layer "F.Cu") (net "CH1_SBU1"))
 (segment (start 28.9458 35.27) (end 30.2309 33.9849) (width 0.2) (layer "F.Cu") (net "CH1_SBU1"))
 (segment (start 32.9731 33.9849) (end 33.5899 34.6017) (width 0.2) (layer "F.Cu") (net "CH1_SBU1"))
 (segment (start 33.5899 34.6017) (end 38.45 34.6017) (width 0.2) (layer "F.Cu") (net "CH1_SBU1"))
 (segment (start 38.0348 50) (end 45.55 50) (width 0.2) (layer "F.Cu") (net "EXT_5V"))
 (segment (start 37.55 42) (end 36.9483 42) (width 0.2) (layer "F.Cu") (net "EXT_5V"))
 (segment (start 43.7966 41.3983) (end 36.9583 41.3983) (width 0.2) (layer "F.Cu") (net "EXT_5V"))
 (segment (start 60.3466 50.6017) (end 60.9483 50) (width 0.2) (layer "F.Cu") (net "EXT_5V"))
 (segment (start 45.1 42) (end 44.3983 42) (width 0.2) (layer "F.Cu") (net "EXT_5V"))
 (segment (start 44.3983 42) (end 43.7966 41.3983) (width 0.2) (layer "F.Cu") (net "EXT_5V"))
 (segment (start 30.81 35.27) (end 36.9483 41.4083) (width 0.2) (layer "F.Cu") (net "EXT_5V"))
 (segment (start 45.55 50) (end 45.55 50.6017) (width 0.2) (layer "F.Cu") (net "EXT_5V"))
 (segment (start 36.9583 41.3983) (end 36.9483 41.4083) (width 0.2) (layer "F.Cu") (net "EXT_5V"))
 (segment (start 36.9483 41.4083) (end 36.9483 42) (width 0.2) (layer "F.Cu") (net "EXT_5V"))
 (segment (start 61.55 50) (end 60.9483 50) (width 0.2) (layer "F.Cu") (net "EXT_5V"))
 (segment (start 45.55 50.6017) (end 60.3466 50.6017) (width 0.2) (layer "F.Cu") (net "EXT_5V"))
 (via (at 38.0348 50) (size 0.6) (drill 0.3) (layers "F.Cu" "B.Cu") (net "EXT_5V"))
 (segment (start 24.46 34) (end 23.19 32.73) (width 0.2) (layer "B.Cu") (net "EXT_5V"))
 (segment (start 30.81 35.27) (end 29.54 34) (width 0.2) (layer "B.Cu") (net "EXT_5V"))
 (segment (start 29.54 34) (end 24.46 34) (width 0.2) (layer "B.Cu") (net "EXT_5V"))
 (segment (start 30.81 35.27) (end 38.0348 42.4948) (width 0.2) (layer "B.Cu") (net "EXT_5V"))
 (segment (start 38.0348 42.4948) (end 38.0348 50) (width 0.2) (layer "B.Cu") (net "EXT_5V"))
 (segment (start 61.05 24.6999) (end 61.05 23.7982) (width 0.2) (layer "F.Cu") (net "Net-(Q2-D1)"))
 (segment (start 60.071 33.1227) (end 60.9483 34) (width 0.2) (layer "F.Cu") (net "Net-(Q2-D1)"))
 (segment (start 61.55 34) (end 60.9483 34) (width 0.2) (layer "F.Cu") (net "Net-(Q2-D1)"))
 (segment (start 59.05 33.1227) (end 60.071 33.1227) (width 0.2) (layer "F.Cu") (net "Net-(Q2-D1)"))
 (segment (start 61.05 23.7982) (end 60.3444 23.7982) (width 0.2) (layer "F.Cu") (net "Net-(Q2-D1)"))
 (via (at 60.3444 23.7982) (size 0.6) (drill 0.3) (layers "F.Cu" "B.Cu") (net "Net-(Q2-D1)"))
 (via (at 59.05 33.1227) (size 0.6) (drill 0.3) (layers "F.Cu" "B.Cu") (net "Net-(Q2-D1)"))
 (segment (start 59.05 25.0926) (end 60.3444 23.7982) (width 0.2) (layer "B.Cu") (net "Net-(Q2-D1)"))
 (segment (start 59.05 33.1227) (end 59.05 25.0926) (width 0.2) (layer "B.Cu") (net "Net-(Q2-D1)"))
 (segment (start 46.45 50) (end 49.8886 50) (width 0.2) (layer "F.Cu") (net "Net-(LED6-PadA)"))
 (segment (start 54 27.05) (end 54.9017 27.05) (width 0.2) (layer "F.Cu") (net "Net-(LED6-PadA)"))
 (segment (start 54.9017 27.05) (end 55.1206 27.05) (width 0.2) (layer "F.Cu") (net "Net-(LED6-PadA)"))
 (via (at 55.1206 27.05) (size 0.6) (drill 0.3) (layers "F.Cu" "B.Cu") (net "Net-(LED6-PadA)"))
 (via (at 49.8886 50) (size 0.6) (drill 0.3) (layers "F.Cu" "B.Cu") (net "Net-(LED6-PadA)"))
 (segment (start 49.8886 32.282) (end 49.8886 50) (width 0.2) (layer "B.Cu") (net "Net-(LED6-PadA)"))
 (segment (start 55.1206 27.05) (end 49.8886 32.282) (width 0.2) (layer "B.Cu") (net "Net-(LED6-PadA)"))
 (segment (start 50.4681 45.4164) (end 54.45 49.3983) (width 0.2) (layer "F.Cu") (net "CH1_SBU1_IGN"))
 (segment (start 35.8764 45.4164) (end 50.4681 45.4164) (width 0.2) (layer "F.Cu") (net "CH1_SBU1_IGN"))
 (segment (start 47.1501 28.2018) (end 45.55 26.6017) (width 0.2) (layer "F.Cu") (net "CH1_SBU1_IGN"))
 (segment (start 45.55 26) (end 45.55 26.6017) (width 0.2) (layer "F.Cu") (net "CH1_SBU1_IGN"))
 (segment (start 56.5603 28.2018) (end 47.1501 28.2018) (width 0.2) (layer "F.Cu") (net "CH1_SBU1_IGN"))
 (segment (start 50.4681 45.4164) (end 50.4999 45.3846) (width 0.2) (layer "F.Cu") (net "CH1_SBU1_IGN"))
 (segment (start 54.45 50) (end 54.45 49.3983) (width 0.2) (layer "F.Cu") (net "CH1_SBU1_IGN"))
 (segment (start 61.05 27.3001) (end 61.05 28.2018) (width 0.2) (layer "F.Cu") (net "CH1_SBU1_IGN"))
 (segment (start 25.73 35.27) (end 35.8764 45.4164) (width 0.2) (layer "F.Cu") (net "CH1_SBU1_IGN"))
 (segment (start 61.05 28.2018) (end 56.5603 28.2018) (width 0.2) (layer "F.Cu") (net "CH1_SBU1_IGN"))
 (via (at 50.4999 45.3846) (size 0.6) (drill 0.3) (layers "F.Cu" "B.Cu") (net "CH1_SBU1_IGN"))
 (via (at 56.5603 28.2018) (size 0.6) (drill 0.3) (layers "F.Cu" "B.Cu") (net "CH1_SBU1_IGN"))
 (segment (start 50.4999 34.2622) (end 56.5603 28.2018) (width 0.2) (layer "B.Cu") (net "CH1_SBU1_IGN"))
 (segment (start 50.4999 45.3846) (end 50.4999 34.2622) (width 0.2) (layer "B.Cu") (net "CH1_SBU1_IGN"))
 (segment (start 34.4205 31.4722) (end 36.9483 34) (width 0.2) (layer "F.Cu") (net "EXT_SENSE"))
 (segment (start 37.55 34) (end 36.9483 34) (width 0.2) (layer "F.Cu") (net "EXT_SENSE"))
 (segment (start 28.27 32.73) (end 29.5278 31.4722) (width 0.2) (layer "F.Cu") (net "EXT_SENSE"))
 (segment (start 29.5278 31.4722) (end 34.4205 31.4722) (width 0.2) (layer "F.Cu") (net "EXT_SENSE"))
 (segment (start 52.9483 50) (end 50.7635 47.8152) (width 0.2) (layer "F.Cu") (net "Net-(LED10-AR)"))
 (segment (start 53.55 50) (end 52.9483 50) (width 0.2) (layer "F.Cu") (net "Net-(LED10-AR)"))
 (segment (start 37.7517 27) (end 37.9567 27) (width 0.2) (layer "F.Cu") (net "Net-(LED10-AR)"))
 (segment (start 37.05 27) (end 37.7517 27) (width 0.2) (layer "F.Cu") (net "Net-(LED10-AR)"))
 (segment (start 50.7635 47.8152) (end 44.55 47.8152) (width 0.2) (layer "F.Cu") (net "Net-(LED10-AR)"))
 (via (at 44.55 47.8152) (size 0.6) (drill 0.3) (layers "F.Cu" "B.Cu") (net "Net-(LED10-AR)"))
 (via (at 37.9567 27) (size 0.6) (drill 0.3) (layers "F.Cu" "B.Cu") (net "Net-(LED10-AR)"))
 (segment (start 44.55 33.5933) (end 37.9567 27) (width 0.2) (layer "B.Cu") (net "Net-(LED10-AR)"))
 (segment (start 44.55 47.8152) (end 44.55 33.5933) (width 0.2) (layer "B.Cu") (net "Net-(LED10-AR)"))
 (segment (start 47.7763 28.828) (end 52.9483 34) (width 0.2) (layer "F.Cu") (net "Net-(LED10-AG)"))
 (segment (start 39.6517 27) (end 41.4797 28.828) (width 0.2) (layer "F.Cu") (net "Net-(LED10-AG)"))
 (segment (start 41.4797 28.828) (end 47.7763 28.828) (width 0.2) (layer "F.Cu") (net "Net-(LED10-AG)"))
 (segment (start 53.55 34) (end 52.9483 34) (width 0.2) (layer "F.Cu") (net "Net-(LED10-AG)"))
 (segment (start 38.95 27) (end 39.6517 27) (width 0.2) (layer "F.Cu") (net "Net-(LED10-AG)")))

